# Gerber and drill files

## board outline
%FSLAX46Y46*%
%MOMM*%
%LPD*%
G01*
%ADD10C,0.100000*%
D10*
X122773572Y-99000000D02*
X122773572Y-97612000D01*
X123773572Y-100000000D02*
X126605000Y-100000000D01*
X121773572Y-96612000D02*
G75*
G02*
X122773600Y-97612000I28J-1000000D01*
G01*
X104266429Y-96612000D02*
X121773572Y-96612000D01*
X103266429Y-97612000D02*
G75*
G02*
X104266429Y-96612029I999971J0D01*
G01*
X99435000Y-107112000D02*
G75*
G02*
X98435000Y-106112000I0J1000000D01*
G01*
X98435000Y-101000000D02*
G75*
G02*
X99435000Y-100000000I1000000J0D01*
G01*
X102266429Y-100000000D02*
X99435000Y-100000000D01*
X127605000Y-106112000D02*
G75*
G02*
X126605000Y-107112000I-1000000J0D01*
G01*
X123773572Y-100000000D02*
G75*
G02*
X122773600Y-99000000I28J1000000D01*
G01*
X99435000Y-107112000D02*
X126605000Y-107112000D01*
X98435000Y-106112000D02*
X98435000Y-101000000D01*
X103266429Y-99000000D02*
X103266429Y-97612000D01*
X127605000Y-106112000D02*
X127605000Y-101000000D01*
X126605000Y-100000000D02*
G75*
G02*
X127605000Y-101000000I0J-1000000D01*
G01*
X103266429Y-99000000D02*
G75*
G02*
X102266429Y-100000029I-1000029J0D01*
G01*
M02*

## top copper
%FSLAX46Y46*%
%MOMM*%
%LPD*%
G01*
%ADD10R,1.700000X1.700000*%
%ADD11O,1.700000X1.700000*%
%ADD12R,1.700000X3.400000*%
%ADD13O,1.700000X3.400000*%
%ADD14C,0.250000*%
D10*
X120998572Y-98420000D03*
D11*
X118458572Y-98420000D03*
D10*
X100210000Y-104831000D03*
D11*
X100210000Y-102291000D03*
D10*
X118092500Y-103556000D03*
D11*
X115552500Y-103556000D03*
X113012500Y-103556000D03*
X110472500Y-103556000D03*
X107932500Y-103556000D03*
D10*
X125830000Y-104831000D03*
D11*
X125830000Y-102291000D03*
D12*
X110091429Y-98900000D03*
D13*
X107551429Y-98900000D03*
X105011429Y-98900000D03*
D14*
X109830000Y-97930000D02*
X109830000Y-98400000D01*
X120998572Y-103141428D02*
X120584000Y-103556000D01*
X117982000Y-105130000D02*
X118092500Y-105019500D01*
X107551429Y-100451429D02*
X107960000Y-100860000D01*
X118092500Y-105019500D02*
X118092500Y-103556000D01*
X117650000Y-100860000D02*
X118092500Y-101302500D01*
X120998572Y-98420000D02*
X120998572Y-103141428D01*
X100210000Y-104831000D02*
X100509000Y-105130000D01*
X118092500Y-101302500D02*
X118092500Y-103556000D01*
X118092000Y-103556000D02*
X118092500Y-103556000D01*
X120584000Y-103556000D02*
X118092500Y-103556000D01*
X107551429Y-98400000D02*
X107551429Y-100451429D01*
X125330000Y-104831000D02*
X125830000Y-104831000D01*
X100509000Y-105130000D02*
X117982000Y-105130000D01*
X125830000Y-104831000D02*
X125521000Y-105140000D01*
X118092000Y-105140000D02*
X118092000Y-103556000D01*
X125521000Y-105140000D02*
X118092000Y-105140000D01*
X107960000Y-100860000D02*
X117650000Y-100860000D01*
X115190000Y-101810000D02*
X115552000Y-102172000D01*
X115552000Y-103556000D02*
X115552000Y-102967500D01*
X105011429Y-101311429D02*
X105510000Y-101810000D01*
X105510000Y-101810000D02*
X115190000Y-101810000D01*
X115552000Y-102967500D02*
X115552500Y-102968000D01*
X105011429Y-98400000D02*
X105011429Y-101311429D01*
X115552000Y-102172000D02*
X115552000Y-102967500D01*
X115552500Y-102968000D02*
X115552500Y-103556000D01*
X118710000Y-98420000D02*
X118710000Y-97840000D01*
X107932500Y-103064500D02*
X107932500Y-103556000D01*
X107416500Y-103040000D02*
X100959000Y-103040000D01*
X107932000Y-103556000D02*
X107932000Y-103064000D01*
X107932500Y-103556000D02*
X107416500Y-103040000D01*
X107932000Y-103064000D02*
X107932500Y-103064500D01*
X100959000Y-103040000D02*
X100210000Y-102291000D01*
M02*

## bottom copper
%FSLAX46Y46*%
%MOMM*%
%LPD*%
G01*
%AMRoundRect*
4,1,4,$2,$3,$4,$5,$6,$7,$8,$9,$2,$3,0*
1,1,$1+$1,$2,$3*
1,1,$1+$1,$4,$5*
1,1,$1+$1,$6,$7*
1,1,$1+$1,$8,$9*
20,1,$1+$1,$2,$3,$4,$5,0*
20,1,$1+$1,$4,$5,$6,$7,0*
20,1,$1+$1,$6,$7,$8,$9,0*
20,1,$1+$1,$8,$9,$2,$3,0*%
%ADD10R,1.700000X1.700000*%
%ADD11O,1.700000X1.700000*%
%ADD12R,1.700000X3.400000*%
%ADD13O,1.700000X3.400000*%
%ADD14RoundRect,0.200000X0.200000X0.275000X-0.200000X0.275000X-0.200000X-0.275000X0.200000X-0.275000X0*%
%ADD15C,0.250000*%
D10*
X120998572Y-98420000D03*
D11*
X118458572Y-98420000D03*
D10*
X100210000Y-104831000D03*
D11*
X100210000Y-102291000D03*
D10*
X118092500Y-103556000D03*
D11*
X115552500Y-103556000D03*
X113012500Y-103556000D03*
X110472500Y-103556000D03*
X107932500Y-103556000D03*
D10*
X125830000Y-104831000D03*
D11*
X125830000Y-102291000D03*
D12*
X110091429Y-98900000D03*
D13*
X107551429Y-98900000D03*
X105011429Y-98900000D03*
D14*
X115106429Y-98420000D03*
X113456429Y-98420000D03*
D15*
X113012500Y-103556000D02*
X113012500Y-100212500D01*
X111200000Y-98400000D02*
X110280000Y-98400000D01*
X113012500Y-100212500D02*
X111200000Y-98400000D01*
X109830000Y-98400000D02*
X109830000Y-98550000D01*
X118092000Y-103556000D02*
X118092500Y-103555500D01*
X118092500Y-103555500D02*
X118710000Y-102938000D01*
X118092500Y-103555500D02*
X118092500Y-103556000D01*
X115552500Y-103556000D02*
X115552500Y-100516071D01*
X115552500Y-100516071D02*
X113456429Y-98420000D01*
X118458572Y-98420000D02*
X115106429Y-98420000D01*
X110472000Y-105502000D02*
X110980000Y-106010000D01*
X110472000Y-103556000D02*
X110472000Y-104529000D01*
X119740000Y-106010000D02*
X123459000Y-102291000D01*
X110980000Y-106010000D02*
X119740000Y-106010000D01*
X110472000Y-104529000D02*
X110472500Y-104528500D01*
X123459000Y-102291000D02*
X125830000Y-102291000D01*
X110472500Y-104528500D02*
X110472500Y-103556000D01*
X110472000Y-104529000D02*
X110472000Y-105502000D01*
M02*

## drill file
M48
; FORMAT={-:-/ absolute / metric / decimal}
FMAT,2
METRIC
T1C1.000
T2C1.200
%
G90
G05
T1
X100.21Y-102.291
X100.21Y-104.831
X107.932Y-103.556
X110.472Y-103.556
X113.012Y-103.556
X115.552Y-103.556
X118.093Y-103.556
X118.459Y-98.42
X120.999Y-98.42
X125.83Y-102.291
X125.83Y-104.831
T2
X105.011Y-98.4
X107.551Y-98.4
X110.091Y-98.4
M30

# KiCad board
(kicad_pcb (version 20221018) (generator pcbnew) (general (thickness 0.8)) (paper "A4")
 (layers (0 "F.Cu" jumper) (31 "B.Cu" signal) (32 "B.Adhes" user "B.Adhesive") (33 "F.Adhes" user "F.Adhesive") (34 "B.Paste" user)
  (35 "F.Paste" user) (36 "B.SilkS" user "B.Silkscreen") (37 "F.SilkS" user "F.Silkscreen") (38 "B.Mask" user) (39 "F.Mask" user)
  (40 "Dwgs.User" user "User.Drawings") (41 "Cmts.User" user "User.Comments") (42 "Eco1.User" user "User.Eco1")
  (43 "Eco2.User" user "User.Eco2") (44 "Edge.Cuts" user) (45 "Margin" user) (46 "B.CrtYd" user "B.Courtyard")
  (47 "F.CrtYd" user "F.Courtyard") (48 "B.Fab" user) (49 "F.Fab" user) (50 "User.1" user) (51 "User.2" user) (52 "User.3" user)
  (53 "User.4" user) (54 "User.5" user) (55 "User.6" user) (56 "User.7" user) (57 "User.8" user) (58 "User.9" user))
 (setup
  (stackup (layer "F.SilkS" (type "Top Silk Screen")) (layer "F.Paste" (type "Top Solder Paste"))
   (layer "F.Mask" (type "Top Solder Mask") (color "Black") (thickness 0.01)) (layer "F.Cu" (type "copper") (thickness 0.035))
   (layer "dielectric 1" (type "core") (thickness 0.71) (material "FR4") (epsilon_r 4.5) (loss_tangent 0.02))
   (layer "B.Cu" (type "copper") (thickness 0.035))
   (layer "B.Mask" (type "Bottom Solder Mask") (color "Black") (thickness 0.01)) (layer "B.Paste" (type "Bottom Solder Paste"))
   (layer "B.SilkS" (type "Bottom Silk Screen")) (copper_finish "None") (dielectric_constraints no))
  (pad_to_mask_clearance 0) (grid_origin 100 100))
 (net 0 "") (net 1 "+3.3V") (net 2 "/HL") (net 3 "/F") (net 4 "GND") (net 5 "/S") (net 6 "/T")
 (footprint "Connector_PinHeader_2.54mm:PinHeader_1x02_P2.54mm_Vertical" (layer "F.Cu") (at 120.998572 98.42 -90)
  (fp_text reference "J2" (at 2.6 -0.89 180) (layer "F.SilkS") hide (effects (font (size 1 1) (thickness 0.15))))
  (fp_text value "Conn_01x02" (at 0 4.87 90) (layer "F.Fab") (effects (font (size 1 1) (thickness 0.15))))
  (pad "1" thru_hole rect (at 0 0 270) (size 1.7 1.7) (drill 1) (layers "*.Cu" "*.Mask") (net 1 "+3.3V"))
  (pad "2" thru_hole oval (at 0 2.54 270) (size 1.7 1.7) (drill 1) (layers "*.Cu" "*.Mask") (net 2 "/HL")))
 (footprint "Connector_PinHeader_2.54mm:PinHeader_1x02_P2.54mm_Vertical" (layer "F.Cu") (at 100.21 104.831 180)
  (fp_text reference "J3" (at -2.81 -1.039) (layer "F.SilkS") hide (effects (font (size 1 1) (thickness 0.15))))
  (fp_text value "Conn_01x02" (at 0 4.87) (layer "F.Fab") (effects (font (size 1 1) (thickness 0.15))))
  (pad "1" thru_hole rect (at 0 0 180) (size 1.7 1.7) (drill 1) (layers "*.Cu" "*.Mask") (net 1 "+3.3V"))
  (pad "2" thru_hole oval (at 0 2.54 180) (size 1.7 1.7) (drill 1) (layers "*.Cu" "*.Mask") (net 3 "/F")))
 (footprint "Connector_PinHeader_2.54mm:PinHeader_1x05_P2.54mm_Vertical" (layer "F.Cu") (at 118.0925 103.556 -90)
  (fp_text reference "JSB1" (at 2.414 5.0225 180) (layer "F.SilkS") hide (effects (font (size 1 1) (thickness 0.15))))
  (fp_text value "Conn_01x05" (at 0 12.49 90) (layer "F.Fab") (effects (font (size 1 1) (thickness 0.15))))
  (pad "1" thru_hole rect (at 0 0 270) (size 1.7 1.7) (drill 1) (layers "*.Cu" "*.Mask") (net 1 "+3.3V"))
  (pad "2" thru_hole oval (at 0 2.54 270) (size 1.7 1.7) (drill 1) (layers "*.Cu" "*.Mask") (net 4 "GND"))
  (pad "3" thru_hole oval (at 0 5.08 270) (size 1.7 1.7) (drill 1) (layers "*.Cu" "*.Mask") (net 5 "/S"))
  (pad "4" thru_hole oval (at 0 7.62 270) (size 1.7 1.7) (drill 1) (layers "*.Cu" "*.Mask") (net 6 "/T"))
  (pad "5" thru_hole oval (at 0 10.16 270) (size 1.7 1.7) (drill 1) (layers "*.Cu" "*.Mask") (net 3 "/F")))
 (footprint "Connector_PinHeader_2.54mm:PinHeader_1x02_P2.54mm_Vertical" (layer "F.Cu") (at 125.83 104.831 180)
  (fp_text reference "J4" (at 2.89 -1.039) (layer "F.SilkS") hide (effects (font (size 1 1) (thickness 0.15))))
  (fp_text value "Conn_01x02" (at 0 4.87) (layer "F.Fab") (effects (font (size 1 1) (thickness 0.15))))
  (pad "1" thru_hole rect (at 0 0 180) (size 1.7 1.7) (drill 1) (layers "*.Cu" "*.Mask") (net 1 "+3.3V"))
  (pad "2" thru_hole oval (at 0 2.54 180) (size 1.7 1.7) (drill 1) (layers "*.Cu" "*.Mask") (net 6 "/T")))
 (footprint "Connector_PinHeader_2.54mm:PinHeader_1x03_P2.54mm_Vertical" (layer "F.Cu") (at 110.091429 98.4 -90)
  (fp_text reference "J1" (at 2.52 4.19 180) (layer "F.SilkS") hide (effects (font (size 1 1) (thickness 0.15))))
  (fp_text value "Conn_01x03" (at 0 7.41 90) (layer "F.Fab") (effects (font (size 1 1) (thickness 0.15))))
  (pad "1" thru_hole rect (at 0 0 270) (size 3.4 1.7) (drill 1.2 (offset 0.5 0)) (layers "*.Cu" "*.Mask") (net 5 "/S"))
  (pad "2" thru_hole oval (at 0 2.54 270) (size 3.4 1.7) (drill 1.2 (offset 0.5 0)) (layers "*.Cu" "*.Mask") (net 1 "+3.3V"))
  (pad "3" thru_hole oval (at 0 5.08 270) (size 3.4 1.7) (drill 1.2 (offset 0.5 0)) (layers "*.Cu" "*.Mask") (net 4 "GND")))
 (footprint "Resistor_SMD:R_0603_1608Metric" (layer "B.Cu") (at 114.281429 98.42 180)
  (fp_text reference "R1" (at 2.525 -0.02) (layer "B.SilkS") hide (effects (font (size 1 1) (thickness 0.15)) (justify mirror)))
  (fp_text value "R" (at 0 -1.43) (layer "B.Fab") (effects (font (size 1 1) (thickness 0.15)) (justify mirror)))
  (pad "1" smd roundrect (at -0.825 0 180) (size 0.8 0.95) (layers "B.Cu" "B.Paste" "B.Mask") (roundrect_rratio 0.25) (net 2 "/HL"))
  (pad "2" smd roundrect (at 0.825 0 180) (size 0.8 0.95) (layers "B.Cu" "B.Paste" "B.Mask") (roundrect_rratio 0.25) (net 4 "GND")))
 (gr_line (start 122.773572 99) (end 122.773572 97.612) (stroke (width 0.1) (type default)) (layer "Edge.Cuts"))
 (gr_line (start 123.773572 100) (end 126.605 100) (stroke (width 0.1) (type default)) (layer "Edge.Cuts"))
 (gr_arc (start 121.773572 96.612) (mid 122.480679 96.904893) (end 122.773572 97.612) (stroke (width 0.1) (type default))
  (layer "Edge.Cuts"))
 (gr_line (start 104.266429 96.612) (end 121.773572 96.612) (stroke (width 0.1) (type default)) (layer "Edge.Cuts"))
 (gr_arc (start 103.266429 97.612) (mid 103.559322 96.904893) (end 104.266429 96.612) (stroke (width 0.1) (type default))
  (layer "Edge.Cuts"))
 (gr_arc (start 99.435 107.112) (mid 98.727893 106.819107) (end 98.435 106.112) (stroke (width 0.1) (type default)) (layer "Edge.Cuts"))
 (gr_arc (start 98.435 101) (mid 98.727893 100.292893) (end 99.435 100) (stroke (width 0.1) (type default)) (layer "Edge.Cuts"))
 (gr_line (start 102.266429 100) (end 99.435 100) (stroke (width 0.1) (type default)) (layer "Edge.Cuts"))
 (gr_arc (start 127.605 106.112) (mid 127.312107 106.819107) (end 126.605 107.112) (stroke (width 0.1) (type default)) (layer "Edge.Cuts"))
 (gr_arc (start 123.773572 100) (mid 123.066465 99.707107) (end 122.773572 99) (stroke (width 0.1) (type default)) (layer "Edge.Cuts"))
 (gr_line (start 99.435 107.112) (end 126.605 107.112) (stroke (width 0.1) (type default)) (layer "Edge.Cuts"))
 (gr_line (start 98.435 106.112) (end 98.435 101) (stroke (width 0.1) (type default)) (layer "Edge.Cuts"))
 (gr_line (start 103.266429 99) (end 103.266429 97.612) (stroke (width 0.1) (type default)) (layer "Edge.Cuts"))
 (gr_line (start 127.605 106.112) (end 127.605 101) (stroke (width 0.1) (type default)) (layer "Edge.Cuts"))
 (gr_arc (start 126.605 100) (mid 127.312107 100.292893) (end 127.605 101) (stroke (width 0.1) (type default)) (layer "Edge.Cuts"))
 (gr_arc (start 103.266429 99) (mid 102.973536 99.707107) (end 102.266429 100) (stroke (width 0.1) (type default)) (layer "Edge.Cuts"))
 (segment (start 109.83 97.93) (end 109.83 98.4) (width 0.25) (layer "F.Cu") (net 5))
 (segment (start 113.0125 103.556) (end 113.0125 100.2125) (width 0.25) (layer "B.Cu") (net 5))
 (segment (start 111.2 98.4) (end 110.28 98.4) (width 0.25) (layer "B.Cu") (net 5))
 (segment (start 113.0125 100.2125) (end 111.2 98.4) (width 0.25) (layer "B.Cu") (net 5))
 (segment (start 109.83 98.4) (end 109.83 98.55) (width 0.25) (layer "B.Cu") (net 5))
 (segment (start 120.998572 103.141428) (end 120.584 103.556) (width 0.25) (layer "F.Cu") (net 1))
 (segment (start 117.982 105.13) (end 118.0925 105.0195) (width 0.25) (layer "F.Cu") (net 1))
 (segment (start 107.551429 100.451429) (end 107.96 100.86) (width 0.25) (layer "F.Cu") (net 1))
 (segment (start 118.0925 105.0195) (end 118.0925 103.556) (width 0.25) (layer "F.Cu") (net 1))
 (segment (start 117.65 100.86) (end 118.0925 101.3025) (width 0.25) (layer "F.Cu") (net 1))
 (segment (start 120.998572 98.42) (end 120.998572 103.141428) (width 0.25) (layer "F.Cu") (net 1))
 (segment (start 100.21 104.831) (end 100.509 105.13) (width 0.25) (layer "F.Cu") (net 1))
 (segment (start 118.0925 101.3025) (end 118.0925 103.556) (width 0.25) (layer "F.Cu") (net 1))
 (segment (start 118.092 103.556) (end 118.0925 103.556) (width 0.25) (layer "F.Cu") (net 1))
 (segment (start 120.584 103.556) (end 118.0925 103.556) (width 0.25) (layer "F.Cu") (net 1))
 (segment (start 107.551429 98.4) (end 107.551429 100.451429) (width 0.25) (layer "F.Cu") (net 1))
 (segment (start 125.33 104.831) (end 125.83 104.831) (width 0.25) (layer "F.Cu") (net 1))
 (segment (start 100.509 105.13) (end 117.982 105.13) (width 0.25) (layer "F.Cu") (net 1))
 (segment (start 125.83 104.831) (end 125.521 105.14) (width 0.25) (layer "F.Cu") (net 1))
 (segment (start 118.092 105.14) (end 118.092 103.556) (width 0.25) (layer "F.Cu") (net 1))
 (segment (start 125.521 105.14) (end 118.092 105.14) (width 0.25) (layer "F.Cu") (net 1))
 (segment (start 107.96 100.86) (end 117.65 100.86) (width 0.25) (layer "F.Cu") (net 1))
 (segment (start 118.092 103.556) (end 118.0925 103.5555) (width 0.25) (layer "B.Cu") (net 1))
 (segment (start 118.0925 103.5555) (end 118.71 102.938) (width 0.25) (layer "B.Cu") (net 1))
 (segment (start 118.0925 103.5555) (end 118.0925 103.556) (width 0.25) (layer "B.Cu") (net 1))
 (segment (start 115.19 101.81) (end 115.552 102.172) (width 0.25) (layer "F.Cu") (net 4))
 (segment (start 115.552 103.556) (end 115.552 102.9675) (width 0.25) (layer "F.Cu") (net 4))
 (segment (start 105.011429 101.311429) (end 105.51 101.81) (width 0.25) (layer "F.Cu") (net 4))
 (segment (start 105.51 101.81) (end 115.19 101.81) (width 0.25) (layer "F.Cu") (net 4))
 (segment (start 115.552 102.9675) (end 115.5525 102.968) (width 0.25) (layer "F.Cu") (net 4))
 (segment (start 105.011429 98.4) (end 105.011429 101.311429) (width 0.25) (layer "F.Cu") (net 4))
 (segment (start 115.552 102.172) (end 115.552 102.9675) (width 0.25) (layer "F.Cu") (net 4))
 (segment (start 115.5525 102.968) (end 115.5525 103.556) (width 0.25) (layer "F.Cu") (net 4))
 (segment (start 115.5525 103.556) (end 115.5525 100.516071) (width 0.25) (layer "B.Cu") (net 4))
 (segment (start 115.5525 100.516071) (end 113.456429 98.42) (width 0.25) (layer "B.Cu") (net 4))
 (segment (start 118.71 98.42) (end 118.71 97.84) (width 0.25) (layer "F.Cu") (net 2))
 (segment (start 118.458572 98.42) (end 115.106429 98.42) (width 0.25) (layer "B.Cu") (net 2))
 (segment (start 107.9325 103.0645) (end 107.9325 103.556) (width 0.25) (layer "F.Cu") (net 3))
 (segment (start 107.4165 103.04) (end 100.959 103.04) (width 0.25) (layer "F.Cu") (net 3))
 (segment (start 107.932 103.556) (end 107.932 103.064) (width 0.25) (layer "F.Cu") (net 3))
 (segment (start 107.9325 103.556) (end 107.4165 103.04) (width 0.25) (layer "F.Cu") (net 3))
 (segment (start 107.932 103.064) (end 107.9325 103.0645) (width 0.25) (layer "F.Cu") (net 3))
 (segment (start 100.959 103.04) (end 100.21 102.291) (width 0.25) (layer "F.Cu") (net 3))
 (segment (start 110.472 105.502) (end 110.98 106.01) (width 0.25) (layer "B.Cu") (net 6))
 (segment (start 110.472 103.556) (end 110.472 104.529) (width 0.25) (layer "B.Cu") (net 6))
 (segment (start 119.74 106.01) (end 123.459 102.291) (width 0.25) (layer "B.Cu") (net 6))
 (segment (start 110.98 106.01) (end 119.74 106.01) (width 0.25) (layer "B.Cu") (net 6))
 (segment (start 110.472 104.529) (end 110.4725 104.5285) (width 0.25) (layer "B.Cu") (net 6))
 (segment (start 123.459 102.291) (end 125.83 102.291) (width 0.25) (layer "B.Cu") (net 6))
 (segment (start 110.4725 104.5285) (end 110.4725 103.556) (width 0.25) (layer "B.Cu") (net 6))
 (segment (start 110.472 104.529) (end 110.472 105.502) (width 0.25) (layer "B.Cu") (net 6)))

